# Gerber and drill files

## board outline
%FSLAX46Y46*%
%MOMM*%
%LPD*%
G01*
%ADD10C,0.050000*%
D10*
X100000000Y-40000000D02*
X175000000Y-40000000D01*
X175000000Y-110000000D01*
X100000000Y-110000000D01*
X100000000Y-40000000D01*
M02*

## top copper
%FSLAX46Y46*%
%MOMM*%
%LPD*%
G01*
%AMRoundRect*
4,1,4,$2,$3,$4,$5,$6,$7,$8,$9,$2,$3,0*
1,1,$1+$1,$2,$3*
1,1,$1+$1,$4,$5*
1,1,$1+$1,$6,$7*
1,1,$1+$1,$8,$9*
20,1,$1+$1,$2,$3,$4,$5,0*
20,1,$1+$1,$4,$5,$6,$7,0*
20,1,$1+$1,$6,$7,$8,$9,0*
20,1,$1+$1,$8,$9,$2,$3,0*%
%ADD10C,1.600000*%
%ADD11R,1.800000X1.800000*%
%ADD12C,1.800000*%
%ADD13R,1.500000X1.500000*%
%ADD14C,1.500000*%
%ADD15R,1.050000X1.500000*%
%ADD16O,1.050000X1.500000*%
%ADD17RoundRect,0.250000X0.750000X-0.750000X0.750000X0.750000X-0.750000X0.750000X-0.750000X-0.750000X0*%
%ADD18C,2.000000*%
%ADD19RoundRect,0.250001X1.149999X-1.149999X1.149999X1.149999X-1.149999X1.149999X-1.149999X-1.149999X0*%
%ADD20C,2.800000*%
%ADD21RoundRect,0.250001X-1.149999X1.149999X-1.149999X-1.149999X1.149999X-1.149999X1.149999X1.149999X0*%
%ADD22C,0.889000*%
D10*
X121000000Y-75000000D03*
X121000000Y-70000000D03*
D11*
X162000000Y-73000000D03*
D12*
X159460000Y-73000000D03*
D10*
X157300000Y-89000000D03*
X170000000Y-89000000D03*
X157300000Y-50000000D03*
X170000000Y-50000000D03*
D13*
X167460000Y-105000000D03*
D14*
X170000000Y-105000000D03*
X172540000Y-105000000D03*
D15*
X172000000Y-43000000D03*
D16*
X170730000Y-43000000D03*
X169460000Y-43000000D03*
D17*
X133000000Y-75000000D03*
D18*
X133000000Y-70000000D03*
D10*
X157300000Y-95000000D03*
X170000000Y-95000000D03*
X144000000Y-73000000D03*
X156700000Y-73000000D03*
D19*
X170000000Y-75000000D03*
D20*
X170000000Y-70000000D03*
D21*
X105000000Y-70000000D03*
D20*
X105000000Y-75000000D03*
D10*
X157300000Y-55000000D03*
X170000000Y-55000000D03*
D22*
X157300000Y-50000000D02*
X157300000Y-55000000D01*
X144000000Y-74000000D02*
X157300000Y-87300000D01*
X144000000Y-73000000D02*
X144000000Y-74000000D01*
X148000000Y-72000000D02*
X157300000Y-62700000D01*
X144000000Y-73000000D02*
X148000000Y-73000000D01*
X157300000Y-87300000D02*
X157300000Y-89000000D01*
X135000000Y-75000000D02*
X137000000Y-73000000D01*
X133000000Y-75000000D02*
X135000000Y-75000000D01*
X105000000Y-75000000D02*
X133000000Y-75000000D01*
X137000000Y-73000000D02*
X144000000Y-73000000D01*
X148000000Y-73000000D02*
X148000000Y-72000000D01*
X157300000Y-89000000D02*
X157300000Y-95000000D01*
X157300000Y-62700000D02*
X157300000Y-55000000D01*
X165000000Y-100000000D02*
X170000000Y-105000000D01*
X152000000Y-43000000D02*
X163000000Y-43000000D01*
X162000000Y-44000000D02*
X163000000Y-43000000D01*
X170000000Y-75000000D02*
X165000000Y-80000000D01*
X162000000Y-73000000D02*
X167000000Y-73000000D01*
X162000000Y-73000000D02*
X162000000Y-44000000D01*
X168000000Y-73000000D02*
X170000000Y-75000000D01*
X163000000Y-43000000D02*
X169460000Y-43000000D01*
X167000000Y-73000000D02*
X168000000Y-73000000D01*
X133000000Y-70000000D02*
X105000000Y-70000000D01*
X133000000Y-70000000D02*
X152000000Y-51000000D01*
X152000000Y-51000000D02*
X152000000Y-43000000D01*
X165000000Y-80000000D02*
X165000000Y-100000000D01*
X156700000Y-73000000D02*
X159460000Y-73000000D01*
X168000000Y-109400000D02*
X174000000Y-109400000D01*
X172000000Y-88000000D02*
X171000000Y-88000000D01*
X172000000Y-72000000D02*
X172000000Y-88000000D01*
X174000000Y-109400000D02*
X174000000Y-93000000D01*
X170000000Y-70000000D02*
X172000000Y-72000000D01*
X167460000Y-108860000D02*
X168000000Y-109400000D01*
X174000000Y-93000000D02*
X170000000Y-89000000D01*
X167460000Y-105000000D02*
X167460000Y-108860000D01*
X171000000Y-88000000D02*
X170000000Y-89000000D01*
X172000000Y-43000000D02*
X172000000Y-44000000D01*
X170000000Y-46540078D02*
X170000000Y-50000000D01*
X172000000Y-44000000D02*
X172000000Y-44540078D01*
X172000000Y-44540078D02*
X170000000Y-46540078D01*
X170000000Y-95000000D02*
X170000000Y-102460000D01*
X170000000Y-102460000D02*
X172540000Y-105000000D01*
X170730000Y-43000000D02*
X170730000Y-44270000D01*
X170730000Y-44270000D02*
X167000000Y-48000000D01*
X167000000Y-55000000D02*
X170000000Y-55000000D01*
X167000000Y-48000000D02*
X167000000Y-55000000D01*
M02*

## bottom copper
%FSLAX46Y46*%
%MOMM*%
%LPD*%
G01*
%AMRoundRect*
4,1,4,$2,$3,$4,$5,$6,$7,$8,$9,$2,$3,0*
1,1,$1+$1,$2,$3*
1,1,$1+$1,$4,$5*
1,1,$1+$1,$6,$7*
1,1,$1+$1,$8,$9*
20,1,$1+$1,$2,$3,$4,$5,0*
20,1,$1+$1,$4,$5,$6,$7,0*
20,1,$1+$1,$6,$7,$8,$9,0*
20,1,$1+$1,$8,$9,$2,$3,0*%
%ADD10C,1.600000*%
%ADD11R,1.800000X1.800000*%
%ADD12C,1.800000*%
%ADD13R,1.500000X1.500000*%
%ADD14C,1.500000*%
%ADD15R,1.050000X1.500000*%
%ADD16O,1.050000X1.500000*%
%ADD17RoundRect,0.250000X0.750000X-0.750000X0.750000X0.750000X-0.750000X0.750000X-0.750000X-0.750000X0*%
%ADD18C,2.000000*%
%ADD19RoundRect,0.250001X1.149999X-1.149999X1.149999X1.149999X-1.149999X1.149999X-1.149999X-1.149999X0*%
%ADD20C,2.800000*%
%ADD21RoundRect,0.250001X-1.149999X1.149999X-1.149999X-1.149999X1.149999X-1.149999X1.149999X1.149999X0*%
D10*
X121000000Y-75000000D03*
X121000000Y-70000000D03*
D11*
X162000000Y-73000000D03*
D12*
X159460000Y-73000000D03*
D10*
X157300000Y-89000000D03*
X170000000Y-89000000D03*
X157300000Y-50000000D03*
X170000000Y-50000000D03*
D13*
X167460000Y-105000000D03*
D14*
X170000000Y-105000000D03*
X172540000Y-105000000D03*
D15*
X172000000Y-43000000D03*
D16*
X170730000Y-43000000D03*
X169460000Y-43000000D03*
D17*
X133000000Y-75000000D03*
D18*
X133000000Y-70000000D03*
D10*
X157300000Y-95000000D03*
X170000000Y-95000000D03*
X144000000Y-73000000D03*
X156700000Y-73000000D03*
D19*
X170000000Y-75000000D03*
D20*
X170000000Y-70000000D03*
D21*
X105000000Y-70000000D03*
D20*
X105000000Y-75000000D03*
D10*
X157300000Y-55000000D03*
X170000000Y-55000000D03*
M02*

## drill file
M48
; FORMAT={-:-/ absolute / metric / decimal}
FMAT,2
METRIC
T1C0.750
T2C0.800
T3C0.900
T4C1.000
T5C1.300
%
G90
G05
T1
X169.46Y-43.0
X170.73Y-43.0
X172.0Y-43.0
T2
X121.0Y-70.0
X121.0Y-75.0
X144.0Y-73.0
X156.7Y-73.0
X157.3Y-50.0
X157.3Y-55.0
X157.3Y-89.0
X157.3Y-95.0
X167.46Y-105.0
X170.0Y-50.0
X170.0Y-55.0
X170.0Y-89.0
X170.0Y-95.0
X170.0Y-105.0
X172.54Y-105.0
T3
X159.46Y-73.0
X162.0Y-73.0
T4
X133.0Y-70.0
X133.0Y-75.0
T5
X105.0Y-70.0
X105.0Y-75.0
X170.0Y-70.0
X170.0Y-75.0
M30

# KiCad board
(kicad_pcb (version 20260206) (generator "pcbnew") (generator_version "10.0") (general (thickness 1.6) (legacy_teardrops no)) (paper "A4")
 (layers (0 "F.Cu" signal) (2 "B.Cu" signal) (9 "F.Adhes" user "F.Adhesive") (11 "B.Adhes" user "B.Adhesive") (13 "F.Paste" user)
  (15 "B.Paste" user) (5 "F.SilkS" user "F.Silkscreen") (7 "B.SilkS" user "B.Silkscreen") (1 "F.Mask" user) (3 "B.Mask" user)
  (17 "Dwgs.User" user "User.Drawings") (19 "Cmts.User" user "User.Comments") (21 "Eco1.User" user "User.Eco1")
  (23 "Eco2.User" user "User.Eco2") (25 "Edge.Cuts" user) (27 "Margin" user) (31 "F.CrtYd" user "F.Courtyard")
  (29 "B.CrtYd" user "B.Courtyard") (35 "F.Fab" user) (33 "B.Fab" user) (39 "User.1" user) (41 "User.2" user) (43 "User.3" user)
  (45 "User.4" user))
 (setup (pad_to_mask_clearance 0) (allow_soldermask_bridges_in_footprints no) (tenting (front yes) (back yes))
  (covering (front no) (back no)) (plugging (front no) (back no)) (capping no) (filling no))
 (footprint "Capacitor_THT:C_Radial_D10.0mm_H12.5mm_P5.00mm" (layer "F.Cu") (at 121 75 90)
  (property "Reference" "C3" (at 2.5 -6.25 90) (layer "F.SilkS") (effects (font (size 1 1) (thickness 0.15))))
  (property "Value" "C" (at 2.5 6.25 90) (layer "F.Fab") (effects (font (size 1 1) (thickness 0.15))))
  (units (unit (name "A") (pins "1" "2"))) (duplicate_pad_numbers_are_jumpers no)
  (pad "1" thru_hole circle (at 0 0 90) (size 1.6 1.6) (drill 0.8) (layers "*.Cu" "*.Mask") (remove_unused_layers no) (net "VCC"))
  (pad "2" thru_hole circle (at 5 0 90) (size 1.6 1.6) (drill 0.8) (layers "*.Cu" "*.Mask") (remove_unused_layers no) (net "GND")))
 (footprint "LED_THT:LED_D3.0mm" (layer "F.Cu") (at 162 73 180)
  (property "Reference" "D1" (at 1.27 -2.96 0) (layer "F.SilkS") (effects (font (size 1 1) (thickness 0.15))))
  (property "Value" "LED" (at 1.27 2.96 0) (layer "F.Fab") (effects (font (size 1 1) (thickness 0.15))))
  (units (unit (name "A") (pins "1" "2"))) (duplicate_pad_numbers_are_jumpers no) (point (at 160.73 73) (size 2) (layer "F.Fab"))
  (pad "1" thru_hole rect (at 0 0 180) (size 1.8 1.8) (drill 0.9) (layers "*.Cu" "*.Mask") (remove_unused_layers no) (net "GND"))
  (pad "2" thru_hole circle (at 2.54 0 180) (size 1.8 1.8) (drill 0.9) (layers "*.Cu" "*.Mask") (remove_unused_layers no) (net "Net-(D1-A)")))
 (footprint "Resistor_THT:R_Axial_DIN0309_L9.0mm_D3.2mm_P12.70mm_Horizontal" (layer "F.Cu") (at 157.3 89)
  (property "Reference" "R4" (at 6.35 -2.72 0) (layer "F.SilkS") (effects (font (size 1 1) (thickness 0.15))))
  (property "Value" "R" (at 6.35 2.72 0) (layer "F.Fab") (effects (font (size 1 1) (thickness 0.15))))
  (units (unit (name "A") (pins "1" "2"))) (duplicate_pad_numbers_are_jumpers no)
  (pad "1" thru_hole circle (at 0 0) (size 1.6 1.6) (drill 0.8) (layers "*.Cu" "*.Mask") (remove_unused_layers no) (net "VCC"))
  (pad "2" thru_hole circle (at 12.7 0) (size 1.6 1.6) (drill 0.8) (layers "*.Cu" "*.Mask") (remove_unused_layers no) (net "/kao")))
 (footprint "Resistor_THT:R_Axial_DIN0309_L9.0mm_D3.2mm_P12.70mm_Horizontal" (layer "F.Cu") (at 157.3 50)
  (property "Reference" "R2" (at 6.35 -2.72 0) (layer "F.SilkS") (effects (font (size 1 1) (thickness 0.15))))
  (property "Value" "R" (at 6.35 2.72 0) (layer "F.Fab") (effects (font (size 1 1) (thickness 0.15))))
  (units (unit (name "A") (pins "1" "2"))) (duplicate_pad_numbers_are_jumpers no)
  (pad "1" thru_hole circle (at 0 0) (size 1.6 1.6) (drill 0.8) (layers "*.Cu" "*.Mask") (remove_unused_layers no) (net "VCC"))
  (pad "2" thru_hole circle (at 12.7 0) (size 1.6 1.6) (drill 0.8) (layers "*.Cu" "*.Mask") (remove_unused_layers no) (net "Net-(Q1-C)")))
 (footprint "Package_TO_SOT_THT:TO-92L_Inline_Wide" (layer "F.Cu") (at 167.46 105)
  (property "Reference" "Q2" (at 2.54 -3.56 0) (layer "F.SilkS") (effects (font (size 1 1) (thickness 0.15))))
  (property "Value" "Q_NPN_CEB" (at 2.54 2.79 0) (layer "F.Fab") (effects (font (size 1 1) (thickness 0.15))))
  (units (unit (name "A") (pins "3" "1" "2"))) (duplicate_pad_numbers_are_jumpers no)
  (pad "1" thru_hole rect (at 0 0) (size 1.5 1.5) (drill 0.8) (layers "*.Cu" "*.Mask") (remove_unused_layers no) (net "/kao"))
  (pad "2" thru_hole circle (at 2.54 0) (size 1.5 1.5) (drill 0.8) (layers "*.Cu" "*.Mask") (remove_unused_layers no) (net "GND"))
  (pad "3" thru_hole circle (at 5.08 0) (size 1.5 1.5) (drill 0.8) (layers "*.Cu" "*.Mask") (remove_unused_layers no) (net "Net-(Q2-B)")))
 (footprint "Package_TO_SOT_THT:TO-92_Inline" (layer "F.Cu") (at 172 43 180)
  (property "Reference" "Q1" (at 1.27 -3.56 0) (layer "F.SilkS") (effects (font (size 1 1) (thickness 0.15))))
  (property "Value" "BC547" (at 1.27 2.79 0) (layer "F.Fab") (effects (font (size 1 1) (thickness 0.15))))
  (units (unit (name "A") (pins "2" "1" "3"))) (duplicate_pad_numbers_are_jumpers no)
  (pad "1" thru_hole rect (at 0 0 180) (size 1.05 1.5) (drill 0.75) (layers "*.Cu" "*.Mask") (remove_unused_layers no) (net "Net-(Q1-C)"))
  (pad "2" thru_hole oval (at 1.27 0 180) (size 1.05 1.5) (drill 0.75) (layers "*.Cu" "*.Mask") (remove_unused_layers no) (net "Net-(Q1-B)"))
  (pad "3" thru_hole oval (at 2.54 0 180) (size 1.05 1.5) (drill 0.75) (layers "*.Cu" "*.Mask") (remove_unused_layers no) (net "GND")))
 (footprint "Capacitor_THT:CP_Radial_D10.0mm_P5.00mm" (layer "F.Cu") (at 133 75 90)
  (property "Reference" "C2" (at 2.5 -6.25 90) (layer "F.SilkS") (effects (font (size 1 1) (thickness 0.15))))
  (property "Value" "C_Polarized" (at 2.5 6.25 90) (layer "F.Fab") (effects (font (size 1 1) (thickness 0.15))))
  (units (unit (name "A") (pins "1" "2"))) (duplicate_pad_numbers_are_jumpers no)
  (pad "1" thru_hole roundrect (at 0 0 90) (size 2 2) (drill 1) (layers "*.Cu" "*.Mask") (remove_unused_layers no) (roundrect_rratio 0.125)
   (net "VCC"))
  (pad "2" thru_hole circle (at 5 0 90) (size 2 2) (drill 1) (layers "*.Cu" "*.Mask") (remove_unused_layers no) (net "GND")))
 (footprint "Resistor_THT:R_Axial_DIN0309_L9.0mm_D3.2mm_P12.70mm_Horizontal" (layer "F.Cu") (at 157.3 95)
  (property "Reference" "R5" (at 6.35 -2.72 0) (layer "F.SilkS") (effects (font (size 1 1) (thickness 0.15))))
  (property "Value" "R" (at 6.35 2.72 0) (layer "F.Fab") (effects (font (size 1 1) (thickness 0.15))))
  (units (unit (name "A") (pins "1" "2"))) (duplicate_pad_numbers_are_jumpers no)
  (pad "1" thru_hole circle (at 0 0) (size 1.6 1.6) (drill 0.8) (layers "*.Cu" "*.Mask") (remove_unused_layers no) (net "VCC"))
  (pad "2" thru_hole circle (at 12.7 0) (size 1.6 1.6) (drill 0.8) (layers "*.Cu" "*.Mask") (remove_unused_layers no) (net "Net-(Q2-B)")))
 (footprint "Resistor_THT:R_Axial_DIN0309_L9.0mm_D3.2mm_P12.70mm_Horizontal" (layer "F.Cu") (at 144 73)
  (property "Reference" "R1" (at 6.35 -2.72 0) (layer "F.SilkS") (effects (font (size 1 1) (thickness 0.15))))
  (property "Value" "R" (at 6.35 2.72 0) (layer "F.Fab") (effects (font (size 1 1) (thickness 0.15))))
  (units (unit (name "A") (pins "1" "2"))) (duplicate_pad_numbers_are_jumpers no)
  (pad "1" thru_hole circle (at 0 0) (size 1.6 1.6) (drill 0.8) (layers "*.Cu" "*.Mask") (remove_unused_layers no) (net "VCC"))
  (pad "2" thru_hole circle (at 12.7 0) (size 1.6 1.6) (drill 0.8) (layers "*.Cu" "*.Mask") (remove_unused_layers no) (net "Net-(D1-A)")))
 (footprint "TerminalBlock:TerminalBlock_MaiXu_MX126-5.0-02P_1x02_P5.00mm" (layer "F.Cu") (at 170 75 90)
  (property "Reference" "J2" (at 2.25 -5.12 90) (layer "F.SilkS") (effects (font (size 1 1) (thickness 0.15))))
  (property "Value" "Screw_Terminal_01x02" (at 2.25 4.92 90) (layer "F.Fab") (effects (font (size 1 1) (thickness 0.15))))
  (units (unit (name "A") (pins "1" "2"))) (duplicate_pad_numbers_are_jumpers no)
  (pad "1" thru_hole roundrect (at 0 0 90) (size 2.8 2.8) (drill 1.3) (layers "*.Cu" "*.Mask") (remove_unused_layers no)
   (roundrect_rratio 0.089286) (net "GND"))
  (pad "2" thru_hole circle (at 5 0 90) (size 2.8 2.8) (drill 1.3) (layers "*.Cu" "*.Mask") (remove_unused_layers no) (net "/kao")))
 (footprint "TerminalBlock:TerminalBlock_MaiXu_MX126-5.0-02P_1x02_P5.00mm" (layer "F.Cu") (at 105 70 -90)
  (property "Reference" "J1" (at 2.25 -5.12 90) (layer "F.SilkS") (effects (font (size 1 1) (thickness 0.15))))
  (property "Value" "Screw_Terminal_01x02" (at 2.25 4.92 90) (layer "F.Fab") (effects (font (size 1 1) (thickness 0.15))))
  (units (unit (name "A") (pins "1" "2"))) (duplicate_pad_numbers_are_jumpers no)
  (pad "1" thru_hole roundrect (at 0 0 270) (size 2.8 2.8) (drill 1.3) (layers "*.Cu" "*.Mask") (remove_unused_layers no)
   (roundrect_rratio 0.089286) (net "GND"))
  (pad "2" thru_hole circle (at 5 0 270) (size 2.8 2.8) (drill 1.3) (layers "*.Cu" "*.Mask") (remove_unused_layers no) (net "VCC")))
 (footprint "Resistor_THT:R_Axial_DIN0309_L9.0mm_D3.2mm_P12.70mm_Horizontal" (layer "F.Cu") (at 157.3 55)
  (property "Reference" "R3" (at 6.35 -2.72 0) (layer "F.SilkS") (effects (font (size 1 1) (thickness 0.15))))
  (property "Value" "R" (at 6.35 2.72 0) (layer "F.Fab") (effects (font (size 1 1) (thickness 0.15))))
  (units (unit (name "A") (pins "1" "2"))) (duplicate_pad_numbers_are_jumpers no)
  (pad "1" thru_hole circle (at 0 0) (size 1.6 1.6) (drill 0.8) (layers "*.Cu" "*.Mask") (remove_unused_layers no) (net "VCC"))
  (pad "2" thru_hole circle (at 12.7 0) (size 1.6 1.6) (drill 0.8) (layers "*.Cu" "*.Mask") (remove_unused_layers no) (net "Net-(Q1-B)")))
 (gr_rect (start 100 40) (end 175 110) (stroke (width 0.05) (type default)) (fill no) (layer "Edge.Cuts"))
 (segment (start 157.3 50) (end 157.3 55) (width 0.889) (layer "F.Cu") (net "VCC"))
 (segment (start 144 74) (end 157.3 87.3) (width 0.889) (layer "F.Cu") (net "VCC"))
 (segment (start 144 73) (end 144 74) (width 0.889) (layer "F.Cu") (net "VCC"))
 (segment (start 148 72) (end 157.3 62.7) (width 0.889) (layer "F.Cu") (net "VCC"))
 (segment (start 144 73) (end 148 73) (width 0.889) (layer "F.Cu") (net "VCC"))
 (segment (start 157.3 87.3) (end 157.3 89) (width 0.889) (layer "F.Cu") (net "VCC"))
 (segment (start 135 75) (end 137 73) (width 0.889) (layer "F.Cu") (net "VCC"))
 (segment (start 133 75) (end 135 75) (width 0.889) (layer "F.Cu") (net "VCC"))
 (segment (start 105 75) (end 133 75) (width 0.889) (layer "F.Cu") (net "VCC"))
 (segment (start 137 73) (end 144 73) (width 0.889) (layer "F.Cu") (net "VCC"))
 (segment (start 148 73) (end 148 72) (width 0.889) (layer "F.Cu") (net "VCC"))
 (segment (start 157.3 89) (end 157.3 95) (width 0.889) (layer "F.Cu") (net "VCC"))
 (segment (start 157.3 62.7) (end 157.3 55) (width 0.889) (layer "F.Cu") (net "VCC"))
 (segment (start 165 100) (end 170 105) (width 0.889) (layer "F.Cu") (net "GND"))
 (segment (start 152 43) (end 163 43) (width 0.889) (layer "F.Cu") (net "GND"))
 (segment (start 162 44) (end 163 43) (width 0.889) (layer "F.Cu") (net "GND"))
 (segment (start 170 75) (end 165 80) (width 0.889) (layer "F.Cu") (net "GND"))
 (segment (start 162 73) (end 167 73) (width 0.889) (layer "F.Cu") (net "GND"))
 (segment (start 162 73) (end 162 44) (width 0.889) (layer "F.Cu") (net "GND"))
 (segment (start 168 73) (end 170 75) (width 0.889) (layer "F.Cu") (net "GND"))
 (segment (start 163 43) (end 169.46 43) (width 0.889) (layer "F.Cu") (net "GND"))
 (segment (start 167 73) (end 168 73) (width 0.889) (layer "F.Cu") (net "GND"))
 (segment (start 133 70) (end 105 70) (width 0.889) (layer "F.Cu") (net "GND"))
 (segment (start 133 70) (end 152 51) (width 0.889) (layer "F.Cu") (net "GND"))
 (segment (start 152 51) (end 152 43) (width 0.889) (layer "F.Cu") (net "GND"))
 (segment (start 165 80) (end 165 100) (width 0.889) (layer "F.Cu") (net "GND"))
 (segment (start 156.7 73) (end 159.46 73) (width 0.889) (layer "F.Cu") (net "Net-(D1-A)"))
 (segment (start 168 109.4) (end 174 109.4) (width 0.889) (layer "F.Cu") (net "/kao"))
 (segment (start 172 88) (end 171 88) (width 0.889) (layer "F.Cu") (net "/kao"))
 (segment (start 172 72) (end 172 88) (width 0.889) (layer "F.Cu") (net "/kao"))
 (segment (start 174 109.4) (end 174 93) (width 0.889) (layer "F.Cu") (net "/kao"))
 (segment (start 170 70) (end 172 72) (width 0.889) (layer "F.Cu") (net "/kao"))
 (segment (start 167.46 108.86) (end 168 109.4) (width 0.889) (layer "F.Cu") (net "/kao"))
 (segment (start 174 93) (end 170 89) (width 0.889) (layer "F.Cu") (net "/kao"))
 (segment (start 167.46 105) (end 167.46 108.86) (width 0.889) (layer "F.Cu") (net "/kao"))
 (segment (start 171 88) (end 170 89) (width 0.889) (layer "F.Cu") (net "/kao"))
 (segment (start 172 43) (end 172 44) (width 0.889) (layer "F.Cu") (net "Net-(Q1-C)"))
 (segment (start 170 46.540078) (end 170 50) (width 0.889) (layer "F.Cu") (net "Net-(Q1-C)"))
 (segment (start 172 44) (end 172 44.540078) (width 0.889) (layer "F.Cu") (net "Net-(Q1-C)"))
 (segment (start 172 44.540078) (end 170 46.540078) (width 0.889) (layer "F.Cu") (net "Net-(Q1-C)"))
 (segment (start 170 95) (end 170 102.46) (width 0.889) (layer "F.Cu") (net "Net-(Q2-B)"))
 (segment (start 170 102.46) (end 172.54 105) (width 0.889) (layer "F.Cu") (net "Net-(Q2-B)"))
 (segment (start 170.73 43) (end 170.73 44.27) (width 0.889) (layer "F.Cu") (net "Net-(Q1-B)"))
 (segment (start 170.73 44.27) (end 167 48) (width 0.889) (layer "F.Cu") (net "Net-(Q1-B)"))
 (segment (start 167 55) (end 170 55) (width 0.889) (layer "F.Cu") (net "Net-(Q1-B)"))
 (segment (start 167 48) (end 167 55) (width 0.889) (layer "F.Cu") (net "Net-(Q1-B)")))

